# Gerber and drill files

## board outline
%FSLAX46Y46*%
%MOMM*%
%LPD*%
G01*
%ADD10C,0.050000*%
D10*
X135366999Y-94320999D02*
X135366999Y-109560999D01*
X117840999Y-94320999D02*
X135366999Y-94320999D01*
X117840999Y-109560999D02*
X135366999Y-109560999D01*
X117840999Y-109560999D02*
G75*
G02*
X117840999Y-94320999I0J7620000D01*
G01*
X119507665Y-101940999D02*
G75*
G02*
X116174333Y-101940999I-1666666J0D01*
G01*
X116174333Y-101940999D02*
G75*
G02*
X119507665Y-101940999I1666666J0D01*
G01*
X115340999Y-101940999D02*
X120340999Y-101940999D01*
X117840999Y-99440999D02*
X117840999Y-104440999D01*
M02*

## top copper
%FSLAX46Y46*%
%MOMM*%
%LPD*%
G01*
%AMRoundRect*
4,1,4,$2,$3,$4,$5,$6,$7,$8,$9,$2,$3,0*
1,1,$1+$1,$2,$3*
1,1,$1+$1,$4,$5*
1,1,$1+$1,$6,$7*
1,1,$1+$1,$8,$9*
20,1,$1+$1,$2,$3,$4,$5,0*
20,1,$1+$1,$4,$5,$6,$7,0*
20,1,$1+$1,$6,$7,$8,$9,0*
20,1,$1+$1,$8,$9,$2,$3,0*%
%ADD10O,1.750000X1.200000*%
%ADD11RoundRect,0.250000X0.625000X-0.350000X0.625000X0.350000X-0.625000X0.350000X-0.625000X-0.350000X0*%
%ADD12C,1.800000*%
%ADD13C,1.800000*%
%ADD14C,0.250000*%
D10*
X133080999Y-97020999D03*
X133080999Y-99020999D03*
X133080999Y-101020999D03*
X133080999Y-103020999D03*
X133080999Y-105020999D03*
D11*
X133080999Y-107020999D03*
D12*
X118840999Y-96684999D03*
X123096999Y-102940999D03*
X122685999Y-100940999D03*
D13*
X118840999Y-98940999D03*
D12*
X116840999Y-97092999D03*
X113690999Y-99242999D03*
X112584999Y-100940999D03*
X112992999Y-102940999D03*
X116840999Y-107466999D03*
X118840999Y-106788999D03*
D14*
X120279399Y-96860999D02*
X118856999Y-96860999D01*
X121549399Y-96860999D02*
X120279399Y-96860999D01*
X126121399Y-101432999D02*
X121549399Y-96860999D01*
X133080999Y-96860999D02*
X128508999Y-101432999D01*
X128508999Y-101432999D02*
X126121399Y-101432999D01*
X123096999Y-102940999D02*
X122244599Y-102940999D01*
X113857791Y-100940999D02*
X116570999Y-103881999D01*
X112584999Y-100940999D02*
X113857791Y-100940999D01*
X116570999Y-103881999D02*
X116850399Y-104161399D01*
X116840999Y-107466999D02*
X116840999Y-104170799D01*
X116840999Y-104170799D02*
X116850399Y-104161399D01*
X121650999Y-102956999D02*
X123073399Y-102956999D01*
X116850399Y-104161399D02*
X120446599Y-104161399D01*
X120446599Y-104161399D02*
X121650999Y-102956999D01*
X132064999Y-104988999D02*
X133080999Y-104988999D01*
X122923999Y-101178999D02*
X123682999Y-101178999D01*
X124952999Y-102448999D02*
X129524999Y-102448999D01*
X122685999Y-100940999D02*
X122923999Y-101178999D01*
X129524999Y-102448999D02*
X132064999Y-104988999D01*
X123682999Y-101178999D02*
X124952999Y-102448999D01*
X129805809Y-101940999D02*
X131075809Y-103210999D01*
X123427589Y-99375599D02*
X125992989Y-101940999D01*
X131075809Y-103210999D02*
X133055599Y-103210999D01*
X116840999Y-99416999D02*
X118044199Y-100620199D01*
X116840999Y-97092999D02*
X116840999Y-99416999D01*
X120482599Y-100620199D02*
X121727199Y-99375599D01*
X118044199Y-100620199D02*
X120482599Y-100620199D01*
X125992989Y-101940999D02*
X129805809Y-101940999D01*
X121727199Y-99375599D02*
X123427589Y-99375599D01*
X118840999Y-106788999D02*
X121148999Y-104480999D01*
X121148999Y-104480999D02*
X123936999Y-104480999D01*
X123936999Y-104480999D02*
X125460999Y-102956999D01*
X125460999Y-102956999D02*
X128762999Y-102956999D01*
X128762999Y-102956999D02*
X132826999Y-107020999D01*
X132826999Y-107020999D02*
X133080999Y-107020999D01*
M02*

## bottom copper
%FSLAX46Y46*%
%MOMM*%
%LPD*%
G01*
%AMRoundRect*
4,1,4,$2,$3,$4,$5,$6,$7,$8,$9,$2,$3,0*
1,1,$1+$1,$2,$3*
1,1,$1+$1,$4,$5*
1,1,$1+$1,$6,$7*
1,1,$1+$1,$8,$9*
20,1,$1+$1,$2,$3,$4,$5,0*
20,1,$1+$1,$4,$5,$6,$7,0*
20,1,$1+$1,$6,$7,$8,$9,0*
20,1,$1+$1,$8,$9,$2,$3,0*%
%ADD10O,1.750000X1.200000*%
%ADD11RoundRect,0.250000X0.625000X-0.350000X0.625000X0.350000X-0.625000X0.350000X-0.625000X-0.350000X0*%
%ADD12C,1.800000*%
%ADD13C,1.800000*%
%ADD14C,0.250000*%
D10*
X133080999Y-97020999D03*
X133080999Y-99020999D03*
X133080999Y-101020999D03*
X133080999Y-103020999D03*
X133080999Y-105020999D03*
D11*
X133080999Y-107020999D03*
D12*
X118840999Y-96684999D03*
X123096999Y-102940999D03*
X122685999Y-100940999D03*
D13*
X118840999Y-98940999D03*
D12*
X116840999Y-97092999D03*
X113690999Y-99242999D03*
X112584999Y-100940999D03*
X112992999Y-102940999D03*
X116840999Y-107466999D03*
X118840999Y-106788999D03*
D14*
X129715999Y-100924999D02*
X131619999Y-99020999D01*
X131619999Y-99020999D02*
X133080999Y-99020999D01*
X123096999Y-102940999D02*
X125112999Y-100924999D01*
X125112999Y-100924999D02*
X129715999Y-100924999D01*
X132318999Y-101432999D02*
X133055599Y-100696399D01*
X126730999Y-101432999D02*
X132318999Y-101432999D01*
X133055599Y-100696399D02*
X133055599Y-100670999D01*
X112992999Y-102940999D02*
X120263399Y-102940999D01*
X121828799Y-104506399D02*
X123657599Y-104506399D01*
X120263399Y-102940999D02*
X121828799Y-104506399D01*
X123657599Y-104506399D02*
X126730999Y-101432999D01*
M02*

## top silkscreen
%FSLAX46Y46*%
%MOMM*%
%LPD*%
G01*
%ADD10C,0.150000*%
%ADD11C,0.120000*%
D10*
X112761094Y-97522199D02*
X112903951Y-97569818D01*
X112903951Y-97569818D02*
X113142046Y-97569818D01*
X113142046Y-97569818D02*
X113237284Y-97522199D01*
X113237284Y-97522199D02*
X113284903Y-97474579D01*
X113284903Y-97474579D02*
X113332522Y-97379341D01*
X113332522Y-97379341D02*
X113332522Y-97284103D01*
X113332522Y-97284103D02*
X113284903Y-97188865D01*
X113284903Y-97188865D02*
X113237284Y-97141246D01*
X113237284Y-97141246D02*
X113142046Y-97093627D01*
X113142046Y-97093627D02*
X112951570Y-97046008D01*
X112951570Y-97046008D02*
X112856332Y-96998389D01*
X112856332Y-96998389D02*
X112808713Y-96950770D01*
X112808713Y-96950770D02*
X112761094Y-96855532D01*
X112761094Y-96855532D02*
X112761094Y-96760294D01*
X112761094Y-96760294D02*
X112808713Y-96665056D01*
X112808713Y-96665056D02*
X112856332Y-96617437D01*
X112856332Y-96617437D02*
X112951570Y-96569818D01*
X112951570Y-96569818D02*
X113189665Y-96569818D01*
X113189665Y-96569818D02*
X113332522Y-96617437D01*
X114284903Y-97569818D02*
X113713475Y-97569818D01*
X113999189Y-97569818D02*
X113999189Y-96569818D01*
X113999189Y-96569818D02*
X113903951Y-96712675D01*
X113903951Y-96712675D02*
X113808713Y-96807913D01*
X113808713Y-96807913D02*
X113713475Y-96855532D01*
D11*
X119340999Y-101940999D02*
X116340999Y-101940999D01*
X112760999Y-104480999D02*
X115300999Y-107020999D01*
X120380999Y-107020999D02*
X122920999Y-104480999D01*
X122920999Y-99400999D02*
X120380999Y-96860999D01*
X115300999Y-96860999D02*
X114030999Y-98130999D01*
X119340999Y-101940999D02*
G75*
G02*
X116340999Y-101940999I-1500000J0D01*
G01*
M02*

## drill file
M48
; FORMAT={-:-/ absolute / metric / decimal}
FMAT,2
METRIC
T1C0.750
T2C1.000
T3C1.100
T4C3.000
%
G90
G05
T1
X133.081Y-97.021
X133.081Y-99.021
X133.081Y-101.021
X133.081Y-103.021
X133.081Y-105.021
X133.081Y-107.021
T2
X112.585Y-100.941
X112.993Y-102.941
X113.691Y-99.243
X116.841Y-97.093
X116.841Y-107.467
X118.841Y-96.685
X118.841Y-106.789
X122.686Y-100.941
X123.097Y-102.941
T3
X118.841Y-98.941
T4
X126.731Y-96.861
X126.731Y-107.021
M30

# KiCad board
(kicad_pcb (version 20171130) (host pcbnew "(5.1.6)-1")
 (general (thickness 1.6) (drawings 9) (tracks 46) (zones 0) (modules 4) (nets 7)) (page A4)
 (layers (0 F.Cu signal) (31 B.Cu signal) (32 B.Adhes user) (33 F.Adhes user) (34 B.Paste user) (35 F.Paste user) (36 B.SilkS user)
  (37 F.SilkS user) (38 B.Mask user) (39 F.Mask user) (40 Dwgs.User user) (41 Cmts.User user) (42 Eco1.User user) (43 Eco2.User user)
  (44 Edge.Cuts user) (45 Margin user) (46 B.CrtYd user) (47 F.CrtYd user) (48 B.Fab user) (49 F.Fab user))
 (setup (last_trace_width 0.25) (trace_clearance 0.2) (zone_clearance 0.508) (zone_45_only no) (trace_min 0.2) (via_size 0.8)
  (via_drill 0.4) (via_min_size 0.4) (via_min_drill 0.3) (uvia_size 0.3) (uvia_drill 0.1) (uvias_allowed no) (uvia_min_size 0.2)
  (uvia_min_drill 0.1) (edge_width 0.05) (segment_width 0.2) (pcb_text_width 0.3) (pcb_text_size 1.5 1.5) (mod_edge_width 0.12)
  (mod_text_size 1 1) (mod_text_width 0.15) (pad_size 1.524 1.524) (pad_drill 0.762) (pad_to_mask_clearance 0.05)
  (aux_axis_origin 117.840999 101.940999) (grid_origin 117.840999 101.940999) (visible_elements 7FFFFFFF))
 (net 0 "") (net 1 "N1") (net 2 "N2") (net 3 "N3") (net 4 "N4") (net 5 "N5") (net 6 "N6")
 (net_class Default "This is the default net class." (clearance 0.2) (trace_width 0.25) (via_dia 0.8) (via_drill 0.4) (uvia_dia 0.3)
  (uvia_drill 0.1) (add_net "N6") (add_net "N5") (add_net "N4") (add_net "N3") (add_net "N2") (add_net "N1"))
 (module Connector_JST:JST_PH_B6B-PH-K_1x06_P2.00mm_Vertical (layer B.Cu) (at 133.080999 107.020999 90)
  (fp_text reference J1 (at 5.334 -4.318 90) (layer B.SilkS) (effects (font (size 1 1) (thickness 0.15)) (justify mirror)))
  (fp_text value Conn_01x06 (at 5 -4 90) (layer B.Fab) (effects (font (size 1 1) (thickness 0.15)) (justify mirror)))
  (pad 6 thru_hole oval (at 10 0 90) (size 1.2 1.75) (drill 0.75) (layers *.Cu *.Mask) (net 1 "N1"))
  (pad 5 thru_hole oval (at 8 0 90) (size 1.2 1.75) (drill 0.75) (layers *.Cu *.Mask) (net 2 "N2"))
  (pad 4 thru_hole oval (at 6 0 90) (size 1.2 1.75) (drill 0.75) (layers *.Cu *.Mask) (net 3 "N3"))
  (pad 3 thru_hole oval (at 4 0 90) (size 1.2 1.75) (drill 0.75) (layers *.Cu *.Mask) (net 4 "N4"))
  (pad 2 thru_hole oval (at 2 0 90) (size 1.2 1.75) (drill 0.75) (layers *.Cu *.Mask) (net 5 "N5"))
  (pad 1 thru_hole roundrect (at 0 0 90) (size 1.2 1.75) (drill 0.75) (layers *.Cu *.Mask) (roundrect_rratio 0.208333) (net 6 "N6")))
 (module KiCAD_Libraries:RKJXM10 (layer F.Cu) (at 117.840999 101.940999)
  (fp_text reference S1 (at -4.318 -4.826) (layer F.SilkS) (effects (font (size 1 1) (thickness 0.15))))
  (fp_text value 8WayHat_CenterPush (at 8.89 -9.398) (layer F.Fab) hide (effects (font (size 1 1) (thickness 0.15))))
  (fp_line (start 1.5 0) (end -1.5 0) (layer F.SilkS) (width 0.12))
  (fp_line (start -5.08 2.54) (end -2.54 5.08) (layer F.SilkS) (width 0.12))
  (fp_line (start 2.54 5.08) (end 5.08 2.54) (layer F.SilkS) (width 0.12))
  (fp_line (start 5.08 -2.54) (end 2.54 -5.08) (layer F.SilkS) (width 0.12))
  (fp_line (start -2.54 -5.08) (end -3.81 -3.81) (layer F.SilkS) (width 0.12))
  (fp_arc (start 0 0) (end -1.5 0) (angle -180) (layer F.SilkS) (width 0.12))
  (pad COM thru_hole circle (at 1 -5.256) (size 1.8 1.8) (drill 1) (layers *.Cu *.Mask) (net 1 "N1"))
  (pad PUSH3 thru_hole circle (at 5.256 1) (size 1.8 1.8) (drill 1) (layers *.Cu *.Mask) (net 2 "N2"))
  (pad B thru_hole circle (at 4.845 -1) (size 1.8 1.8) (drill 1) (layers *.Cu *.Mask) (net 5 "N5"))
  (pad "" np_thru_hole circle (at 1 -3) (size 1.8 1.8) (drill 1.1) (layers *.Cu *.Mask))
  (pad C thru_hole circle (at -1 -4.848) (size 1.8 1.8) (drill 1) (layers *.Cu *.Mask) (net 4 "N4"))
  (pad GND thru_hole circle (at -4.15 -2.698) (size 1.8 1.8) (drill 1) (layers *.Cu *.Mask))
  (pad PUSH1 thru_hole circle (at -5.256 -1) (size 1.8 1.8) (drill 1) (layers *.Cu *.Mask) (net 2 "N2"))
  (pad D thru_hole circle (at -4.848 1) (size 1.8 1.8) (drill 1) (layers *.Cu *.Mask) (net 3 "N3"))
  (pad PUSH2 thru_hole circle (at -1 5.526) (size 1.8 1.8) (drill 1) (layers *.Cu *.Mask) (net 2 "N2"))
  (pad A thru_hole circle (at 1 4.848) (size 1.8 1.8) (drill 1) (layers *.Cu *.Mask) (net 6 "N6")))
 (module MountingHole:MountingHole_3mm (layer B.Cu) (at 126.730999 107.020999)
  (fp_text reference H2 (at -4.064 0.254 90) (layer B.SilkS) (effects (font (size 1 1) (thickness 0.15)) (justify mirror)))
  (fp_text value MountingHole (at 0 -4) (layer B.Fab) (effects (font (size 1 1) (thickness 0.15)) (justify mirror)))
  (pad 1 np_thru_hole circle (at 0 0) (size 3 3) (drill 3) (layers *.Cu *.Mask)))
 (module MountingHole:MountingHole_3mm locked (layer B.Cu) (at 126.730999 96.860999)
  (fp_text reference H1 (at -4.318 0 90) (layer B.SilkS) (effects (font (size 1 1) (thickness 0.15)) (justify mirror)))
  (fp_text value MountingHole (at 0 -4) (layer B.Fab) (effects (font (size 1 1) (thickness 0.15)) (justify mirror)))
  (pad 1 np_thru_hole circle (at 0 0) (size 3 3) (drill 3) (layers *.Cu *.Mask)))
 (gr_line (start 135.366999 94.320999) (end 135.366999 109.560999) (layer Edge.Cuts) (width 0.05))
 (gr_line (start 117.840999 94.320999) (end 135.366999 94.320999) (layer Edge.Cuts) (width 0.05))
 (gr_line (start 117.840999 109.560999) (end 135.366999 109.560999) (layer Edge.Cuts) (width 0.05))
 (gr_arc (start 117.840999 101.940999) (end 117.840999 94.320999) (angle -180) (layer Edge.Cuts) (width 0.05))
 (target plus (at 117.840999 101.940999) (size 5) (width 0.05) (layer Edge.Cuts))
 (segment (start 120.279399 96.860999) (end 118.856999 96.860999) (width 0.25) (layer F.Cu) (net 1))
 (segment (start 121.549399 96.860999) (end 120.279399 96.860999) (width 0.25) (layer F.Cu) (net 1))
 (segment (start 126.121399 101.432999) (end 121.549399 96.860999) (width 0.25) (layer F.Cu) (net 1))
 (segment (start 133.080999 96.860999) (end 128.508999 101.432999) (width 0.25) (layer F.Cu) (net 1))
 (segment (start 128.508999 101.432999) (end 126.121399 101.432999) (width 0.25) (layer F.Cu) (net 1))
 (segment (start 123.096999 102.940999) (end 122.244599 102.940999) (width 0.25) (layer F.Cu) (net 2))
 (segment (start 113.857791 100.940999) (end 116.570999 103.881999) (width 0.25) (layer F.Cu) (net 2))
 (segment (start 112.584999 100.940999) (end 113.857791 100.940999) (width 0.25) (layer F.Cu) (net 2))
 (segment (start 116.570999 103.881999) (end 116.850399 104.161399) (width 0.25) (layer F.Cu) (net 2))
 (segment (start 116.840999 107.466999) (end 116.840999 104.170799) (width 0.25) (layer F.Cu) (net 2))
 (segment (start 116.840999 104.170799) (end 116.850399 104.161399) (width 0.25) (layer F.Cu) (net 2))
 (segment (start 121.650999 102.956999) (end 123.073399 102.956999) (width 0.25) (layer F.Cu) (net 2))
 (segment (start 116.850399 104.161399) (end 120.446599 104.161399) (width 0.25) (layer F.Cu) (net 2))
 (segment (start 120.446599 104.161399) (end 121.650999 102.956999) (width 0.25) (layer F.Cu) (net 2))
 (segment (start 129.715999 100.924999) (end 131.619999 99.020999) (width 0.25) (layer B.Cu) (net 2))
 (segment (start 131.619999 99.020999) (end 133.080999 99.020999) (width 0.25) (layer B.Cu) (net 2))
 (segment (start 123.096999 102.940999) (end 125.112999 100.924999) (width 0.25) (layer B.Cu) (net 2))
 (segment (start 125.112999 100.924999) (end 129.715999 100.924999) (width 0.25) (layer B.Cu) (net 2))
 (segment (start 132.064999 104.988999) (end 133.080999 104.988999) (width 0.25) (layer F.Cu) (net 5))
 (segment (start 122.923999 101.178999) (end 123.682999 101.178999) (width 0.25) (layer F.Cu) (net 5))
 (segment (start 124.952999 102.448999) (end 129.524999 102.448999) (width 0.25) (layer F.Cu) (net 5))
 (segment (start 122.685999 100.940999) (end 122.923999 101.178999) (width 0.25) (layer F.Cu) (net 5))
 (segment (start 129.524999 102.448999) (end 132.064999 104.988999) (width 0.25) (layer F.Cu) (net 5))
 (segment (start 123.682999 101.178999) (end 124.952999 102.448999) (width 0.25) (layer F.Cu) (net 5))
 (segment (start 129.805809 101.940999) (end 131.075809 103.210999) (width 0.25) (layer F.Cu) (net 4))
 (segment (start 123.427589 99.375599) (end 125.992989 101.940999) (width 0.25) (layer F.Cu) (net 4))
 (segment (start 131.075809 103.210999) (end 133.055599 103.210999) (width 0.25) (layer F.Cu) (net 4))
 (segment (start 116.840999 99.416999) (end 118.044199 100.620199) (width 0.25) (layer F.Cu) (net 4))
 (segment (start 116.840999 97.092999) (end 116.840999 99.416999) (width 0.25) (layer F.Cu) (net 4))
 (segment (start 120.482599 100.620199) (end 121.727199 99.375599) (width 0.25) (layer F.Cu) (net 4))
 (segment (start 118.044199 100.620199) (end 120.482599 100.620199) (width 0.25) (layer F.Cu) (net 4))
 (segment (start 125.992989 101.940999) (end 129.805809 101.940999) (width 0.25) (layer F.Cu) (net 4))
 (segment (start 121.727199 99.375599) (end 123.427589 99.375599) (width 0.25) (layer F.Cu) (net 4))
 (segment (start 132.318999 101.432999) (end 133.055599 100.696399) (width 0.25) (layer B.Cu) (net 3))
 (segment (start 126.730999 101.432999) (end 132.318999 101.432999) (width 0.25) (layer B.Cu) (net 3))
 (segment (start 133.055599 100.696399) (end 133.055599 100.670999) (width 0.25) (layer B.Cu) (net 3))
 (segment (start 112.992999 102.940999) (end 120.263399 102.940999) (width 0.25) (layer B.Cu) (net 3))
 (segment (start 121.828799 104.506399) (end 123.657599 104.506399) (width 0.25) (layer B.Cu) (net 3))
 (segment (start 120.263399 102.940999) (end 121.828799 104.506399) (width 0.25) (layer B.Cu) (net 3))
 (segment (start 123.657599 104.506399) (end 126.730999 101.432999) (width 0.25) (layer B.Cu) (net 3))
 (segment (start 118.840999 106.788999) (end 121.148999 104.480999) (width 0.25) (layer F.Cu) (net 6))
 (segment (start 121.148999 104.480999) (end 123.936999 104.480999) (width 0.25) (layer F.Cu) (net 6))
 (segment (start 123.936999 104.480999) (end 125.460999 102.956999) (width 0.25) (layer F.Cu) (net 6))
 (segment (start 125.460999 102.956999) (end 128.762999 102.956999) (width 0.25) (layer F.Cu) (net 6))
 (segment (start 128.762999 102.956999) (end 132.826999 107.020999) (width 0.25) (layer F.Cu) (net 6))
 (segment (start 132.826999 107.020999) (end 133.080999 107.020999) (width 0.25) (layer F.Cu) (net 6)))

